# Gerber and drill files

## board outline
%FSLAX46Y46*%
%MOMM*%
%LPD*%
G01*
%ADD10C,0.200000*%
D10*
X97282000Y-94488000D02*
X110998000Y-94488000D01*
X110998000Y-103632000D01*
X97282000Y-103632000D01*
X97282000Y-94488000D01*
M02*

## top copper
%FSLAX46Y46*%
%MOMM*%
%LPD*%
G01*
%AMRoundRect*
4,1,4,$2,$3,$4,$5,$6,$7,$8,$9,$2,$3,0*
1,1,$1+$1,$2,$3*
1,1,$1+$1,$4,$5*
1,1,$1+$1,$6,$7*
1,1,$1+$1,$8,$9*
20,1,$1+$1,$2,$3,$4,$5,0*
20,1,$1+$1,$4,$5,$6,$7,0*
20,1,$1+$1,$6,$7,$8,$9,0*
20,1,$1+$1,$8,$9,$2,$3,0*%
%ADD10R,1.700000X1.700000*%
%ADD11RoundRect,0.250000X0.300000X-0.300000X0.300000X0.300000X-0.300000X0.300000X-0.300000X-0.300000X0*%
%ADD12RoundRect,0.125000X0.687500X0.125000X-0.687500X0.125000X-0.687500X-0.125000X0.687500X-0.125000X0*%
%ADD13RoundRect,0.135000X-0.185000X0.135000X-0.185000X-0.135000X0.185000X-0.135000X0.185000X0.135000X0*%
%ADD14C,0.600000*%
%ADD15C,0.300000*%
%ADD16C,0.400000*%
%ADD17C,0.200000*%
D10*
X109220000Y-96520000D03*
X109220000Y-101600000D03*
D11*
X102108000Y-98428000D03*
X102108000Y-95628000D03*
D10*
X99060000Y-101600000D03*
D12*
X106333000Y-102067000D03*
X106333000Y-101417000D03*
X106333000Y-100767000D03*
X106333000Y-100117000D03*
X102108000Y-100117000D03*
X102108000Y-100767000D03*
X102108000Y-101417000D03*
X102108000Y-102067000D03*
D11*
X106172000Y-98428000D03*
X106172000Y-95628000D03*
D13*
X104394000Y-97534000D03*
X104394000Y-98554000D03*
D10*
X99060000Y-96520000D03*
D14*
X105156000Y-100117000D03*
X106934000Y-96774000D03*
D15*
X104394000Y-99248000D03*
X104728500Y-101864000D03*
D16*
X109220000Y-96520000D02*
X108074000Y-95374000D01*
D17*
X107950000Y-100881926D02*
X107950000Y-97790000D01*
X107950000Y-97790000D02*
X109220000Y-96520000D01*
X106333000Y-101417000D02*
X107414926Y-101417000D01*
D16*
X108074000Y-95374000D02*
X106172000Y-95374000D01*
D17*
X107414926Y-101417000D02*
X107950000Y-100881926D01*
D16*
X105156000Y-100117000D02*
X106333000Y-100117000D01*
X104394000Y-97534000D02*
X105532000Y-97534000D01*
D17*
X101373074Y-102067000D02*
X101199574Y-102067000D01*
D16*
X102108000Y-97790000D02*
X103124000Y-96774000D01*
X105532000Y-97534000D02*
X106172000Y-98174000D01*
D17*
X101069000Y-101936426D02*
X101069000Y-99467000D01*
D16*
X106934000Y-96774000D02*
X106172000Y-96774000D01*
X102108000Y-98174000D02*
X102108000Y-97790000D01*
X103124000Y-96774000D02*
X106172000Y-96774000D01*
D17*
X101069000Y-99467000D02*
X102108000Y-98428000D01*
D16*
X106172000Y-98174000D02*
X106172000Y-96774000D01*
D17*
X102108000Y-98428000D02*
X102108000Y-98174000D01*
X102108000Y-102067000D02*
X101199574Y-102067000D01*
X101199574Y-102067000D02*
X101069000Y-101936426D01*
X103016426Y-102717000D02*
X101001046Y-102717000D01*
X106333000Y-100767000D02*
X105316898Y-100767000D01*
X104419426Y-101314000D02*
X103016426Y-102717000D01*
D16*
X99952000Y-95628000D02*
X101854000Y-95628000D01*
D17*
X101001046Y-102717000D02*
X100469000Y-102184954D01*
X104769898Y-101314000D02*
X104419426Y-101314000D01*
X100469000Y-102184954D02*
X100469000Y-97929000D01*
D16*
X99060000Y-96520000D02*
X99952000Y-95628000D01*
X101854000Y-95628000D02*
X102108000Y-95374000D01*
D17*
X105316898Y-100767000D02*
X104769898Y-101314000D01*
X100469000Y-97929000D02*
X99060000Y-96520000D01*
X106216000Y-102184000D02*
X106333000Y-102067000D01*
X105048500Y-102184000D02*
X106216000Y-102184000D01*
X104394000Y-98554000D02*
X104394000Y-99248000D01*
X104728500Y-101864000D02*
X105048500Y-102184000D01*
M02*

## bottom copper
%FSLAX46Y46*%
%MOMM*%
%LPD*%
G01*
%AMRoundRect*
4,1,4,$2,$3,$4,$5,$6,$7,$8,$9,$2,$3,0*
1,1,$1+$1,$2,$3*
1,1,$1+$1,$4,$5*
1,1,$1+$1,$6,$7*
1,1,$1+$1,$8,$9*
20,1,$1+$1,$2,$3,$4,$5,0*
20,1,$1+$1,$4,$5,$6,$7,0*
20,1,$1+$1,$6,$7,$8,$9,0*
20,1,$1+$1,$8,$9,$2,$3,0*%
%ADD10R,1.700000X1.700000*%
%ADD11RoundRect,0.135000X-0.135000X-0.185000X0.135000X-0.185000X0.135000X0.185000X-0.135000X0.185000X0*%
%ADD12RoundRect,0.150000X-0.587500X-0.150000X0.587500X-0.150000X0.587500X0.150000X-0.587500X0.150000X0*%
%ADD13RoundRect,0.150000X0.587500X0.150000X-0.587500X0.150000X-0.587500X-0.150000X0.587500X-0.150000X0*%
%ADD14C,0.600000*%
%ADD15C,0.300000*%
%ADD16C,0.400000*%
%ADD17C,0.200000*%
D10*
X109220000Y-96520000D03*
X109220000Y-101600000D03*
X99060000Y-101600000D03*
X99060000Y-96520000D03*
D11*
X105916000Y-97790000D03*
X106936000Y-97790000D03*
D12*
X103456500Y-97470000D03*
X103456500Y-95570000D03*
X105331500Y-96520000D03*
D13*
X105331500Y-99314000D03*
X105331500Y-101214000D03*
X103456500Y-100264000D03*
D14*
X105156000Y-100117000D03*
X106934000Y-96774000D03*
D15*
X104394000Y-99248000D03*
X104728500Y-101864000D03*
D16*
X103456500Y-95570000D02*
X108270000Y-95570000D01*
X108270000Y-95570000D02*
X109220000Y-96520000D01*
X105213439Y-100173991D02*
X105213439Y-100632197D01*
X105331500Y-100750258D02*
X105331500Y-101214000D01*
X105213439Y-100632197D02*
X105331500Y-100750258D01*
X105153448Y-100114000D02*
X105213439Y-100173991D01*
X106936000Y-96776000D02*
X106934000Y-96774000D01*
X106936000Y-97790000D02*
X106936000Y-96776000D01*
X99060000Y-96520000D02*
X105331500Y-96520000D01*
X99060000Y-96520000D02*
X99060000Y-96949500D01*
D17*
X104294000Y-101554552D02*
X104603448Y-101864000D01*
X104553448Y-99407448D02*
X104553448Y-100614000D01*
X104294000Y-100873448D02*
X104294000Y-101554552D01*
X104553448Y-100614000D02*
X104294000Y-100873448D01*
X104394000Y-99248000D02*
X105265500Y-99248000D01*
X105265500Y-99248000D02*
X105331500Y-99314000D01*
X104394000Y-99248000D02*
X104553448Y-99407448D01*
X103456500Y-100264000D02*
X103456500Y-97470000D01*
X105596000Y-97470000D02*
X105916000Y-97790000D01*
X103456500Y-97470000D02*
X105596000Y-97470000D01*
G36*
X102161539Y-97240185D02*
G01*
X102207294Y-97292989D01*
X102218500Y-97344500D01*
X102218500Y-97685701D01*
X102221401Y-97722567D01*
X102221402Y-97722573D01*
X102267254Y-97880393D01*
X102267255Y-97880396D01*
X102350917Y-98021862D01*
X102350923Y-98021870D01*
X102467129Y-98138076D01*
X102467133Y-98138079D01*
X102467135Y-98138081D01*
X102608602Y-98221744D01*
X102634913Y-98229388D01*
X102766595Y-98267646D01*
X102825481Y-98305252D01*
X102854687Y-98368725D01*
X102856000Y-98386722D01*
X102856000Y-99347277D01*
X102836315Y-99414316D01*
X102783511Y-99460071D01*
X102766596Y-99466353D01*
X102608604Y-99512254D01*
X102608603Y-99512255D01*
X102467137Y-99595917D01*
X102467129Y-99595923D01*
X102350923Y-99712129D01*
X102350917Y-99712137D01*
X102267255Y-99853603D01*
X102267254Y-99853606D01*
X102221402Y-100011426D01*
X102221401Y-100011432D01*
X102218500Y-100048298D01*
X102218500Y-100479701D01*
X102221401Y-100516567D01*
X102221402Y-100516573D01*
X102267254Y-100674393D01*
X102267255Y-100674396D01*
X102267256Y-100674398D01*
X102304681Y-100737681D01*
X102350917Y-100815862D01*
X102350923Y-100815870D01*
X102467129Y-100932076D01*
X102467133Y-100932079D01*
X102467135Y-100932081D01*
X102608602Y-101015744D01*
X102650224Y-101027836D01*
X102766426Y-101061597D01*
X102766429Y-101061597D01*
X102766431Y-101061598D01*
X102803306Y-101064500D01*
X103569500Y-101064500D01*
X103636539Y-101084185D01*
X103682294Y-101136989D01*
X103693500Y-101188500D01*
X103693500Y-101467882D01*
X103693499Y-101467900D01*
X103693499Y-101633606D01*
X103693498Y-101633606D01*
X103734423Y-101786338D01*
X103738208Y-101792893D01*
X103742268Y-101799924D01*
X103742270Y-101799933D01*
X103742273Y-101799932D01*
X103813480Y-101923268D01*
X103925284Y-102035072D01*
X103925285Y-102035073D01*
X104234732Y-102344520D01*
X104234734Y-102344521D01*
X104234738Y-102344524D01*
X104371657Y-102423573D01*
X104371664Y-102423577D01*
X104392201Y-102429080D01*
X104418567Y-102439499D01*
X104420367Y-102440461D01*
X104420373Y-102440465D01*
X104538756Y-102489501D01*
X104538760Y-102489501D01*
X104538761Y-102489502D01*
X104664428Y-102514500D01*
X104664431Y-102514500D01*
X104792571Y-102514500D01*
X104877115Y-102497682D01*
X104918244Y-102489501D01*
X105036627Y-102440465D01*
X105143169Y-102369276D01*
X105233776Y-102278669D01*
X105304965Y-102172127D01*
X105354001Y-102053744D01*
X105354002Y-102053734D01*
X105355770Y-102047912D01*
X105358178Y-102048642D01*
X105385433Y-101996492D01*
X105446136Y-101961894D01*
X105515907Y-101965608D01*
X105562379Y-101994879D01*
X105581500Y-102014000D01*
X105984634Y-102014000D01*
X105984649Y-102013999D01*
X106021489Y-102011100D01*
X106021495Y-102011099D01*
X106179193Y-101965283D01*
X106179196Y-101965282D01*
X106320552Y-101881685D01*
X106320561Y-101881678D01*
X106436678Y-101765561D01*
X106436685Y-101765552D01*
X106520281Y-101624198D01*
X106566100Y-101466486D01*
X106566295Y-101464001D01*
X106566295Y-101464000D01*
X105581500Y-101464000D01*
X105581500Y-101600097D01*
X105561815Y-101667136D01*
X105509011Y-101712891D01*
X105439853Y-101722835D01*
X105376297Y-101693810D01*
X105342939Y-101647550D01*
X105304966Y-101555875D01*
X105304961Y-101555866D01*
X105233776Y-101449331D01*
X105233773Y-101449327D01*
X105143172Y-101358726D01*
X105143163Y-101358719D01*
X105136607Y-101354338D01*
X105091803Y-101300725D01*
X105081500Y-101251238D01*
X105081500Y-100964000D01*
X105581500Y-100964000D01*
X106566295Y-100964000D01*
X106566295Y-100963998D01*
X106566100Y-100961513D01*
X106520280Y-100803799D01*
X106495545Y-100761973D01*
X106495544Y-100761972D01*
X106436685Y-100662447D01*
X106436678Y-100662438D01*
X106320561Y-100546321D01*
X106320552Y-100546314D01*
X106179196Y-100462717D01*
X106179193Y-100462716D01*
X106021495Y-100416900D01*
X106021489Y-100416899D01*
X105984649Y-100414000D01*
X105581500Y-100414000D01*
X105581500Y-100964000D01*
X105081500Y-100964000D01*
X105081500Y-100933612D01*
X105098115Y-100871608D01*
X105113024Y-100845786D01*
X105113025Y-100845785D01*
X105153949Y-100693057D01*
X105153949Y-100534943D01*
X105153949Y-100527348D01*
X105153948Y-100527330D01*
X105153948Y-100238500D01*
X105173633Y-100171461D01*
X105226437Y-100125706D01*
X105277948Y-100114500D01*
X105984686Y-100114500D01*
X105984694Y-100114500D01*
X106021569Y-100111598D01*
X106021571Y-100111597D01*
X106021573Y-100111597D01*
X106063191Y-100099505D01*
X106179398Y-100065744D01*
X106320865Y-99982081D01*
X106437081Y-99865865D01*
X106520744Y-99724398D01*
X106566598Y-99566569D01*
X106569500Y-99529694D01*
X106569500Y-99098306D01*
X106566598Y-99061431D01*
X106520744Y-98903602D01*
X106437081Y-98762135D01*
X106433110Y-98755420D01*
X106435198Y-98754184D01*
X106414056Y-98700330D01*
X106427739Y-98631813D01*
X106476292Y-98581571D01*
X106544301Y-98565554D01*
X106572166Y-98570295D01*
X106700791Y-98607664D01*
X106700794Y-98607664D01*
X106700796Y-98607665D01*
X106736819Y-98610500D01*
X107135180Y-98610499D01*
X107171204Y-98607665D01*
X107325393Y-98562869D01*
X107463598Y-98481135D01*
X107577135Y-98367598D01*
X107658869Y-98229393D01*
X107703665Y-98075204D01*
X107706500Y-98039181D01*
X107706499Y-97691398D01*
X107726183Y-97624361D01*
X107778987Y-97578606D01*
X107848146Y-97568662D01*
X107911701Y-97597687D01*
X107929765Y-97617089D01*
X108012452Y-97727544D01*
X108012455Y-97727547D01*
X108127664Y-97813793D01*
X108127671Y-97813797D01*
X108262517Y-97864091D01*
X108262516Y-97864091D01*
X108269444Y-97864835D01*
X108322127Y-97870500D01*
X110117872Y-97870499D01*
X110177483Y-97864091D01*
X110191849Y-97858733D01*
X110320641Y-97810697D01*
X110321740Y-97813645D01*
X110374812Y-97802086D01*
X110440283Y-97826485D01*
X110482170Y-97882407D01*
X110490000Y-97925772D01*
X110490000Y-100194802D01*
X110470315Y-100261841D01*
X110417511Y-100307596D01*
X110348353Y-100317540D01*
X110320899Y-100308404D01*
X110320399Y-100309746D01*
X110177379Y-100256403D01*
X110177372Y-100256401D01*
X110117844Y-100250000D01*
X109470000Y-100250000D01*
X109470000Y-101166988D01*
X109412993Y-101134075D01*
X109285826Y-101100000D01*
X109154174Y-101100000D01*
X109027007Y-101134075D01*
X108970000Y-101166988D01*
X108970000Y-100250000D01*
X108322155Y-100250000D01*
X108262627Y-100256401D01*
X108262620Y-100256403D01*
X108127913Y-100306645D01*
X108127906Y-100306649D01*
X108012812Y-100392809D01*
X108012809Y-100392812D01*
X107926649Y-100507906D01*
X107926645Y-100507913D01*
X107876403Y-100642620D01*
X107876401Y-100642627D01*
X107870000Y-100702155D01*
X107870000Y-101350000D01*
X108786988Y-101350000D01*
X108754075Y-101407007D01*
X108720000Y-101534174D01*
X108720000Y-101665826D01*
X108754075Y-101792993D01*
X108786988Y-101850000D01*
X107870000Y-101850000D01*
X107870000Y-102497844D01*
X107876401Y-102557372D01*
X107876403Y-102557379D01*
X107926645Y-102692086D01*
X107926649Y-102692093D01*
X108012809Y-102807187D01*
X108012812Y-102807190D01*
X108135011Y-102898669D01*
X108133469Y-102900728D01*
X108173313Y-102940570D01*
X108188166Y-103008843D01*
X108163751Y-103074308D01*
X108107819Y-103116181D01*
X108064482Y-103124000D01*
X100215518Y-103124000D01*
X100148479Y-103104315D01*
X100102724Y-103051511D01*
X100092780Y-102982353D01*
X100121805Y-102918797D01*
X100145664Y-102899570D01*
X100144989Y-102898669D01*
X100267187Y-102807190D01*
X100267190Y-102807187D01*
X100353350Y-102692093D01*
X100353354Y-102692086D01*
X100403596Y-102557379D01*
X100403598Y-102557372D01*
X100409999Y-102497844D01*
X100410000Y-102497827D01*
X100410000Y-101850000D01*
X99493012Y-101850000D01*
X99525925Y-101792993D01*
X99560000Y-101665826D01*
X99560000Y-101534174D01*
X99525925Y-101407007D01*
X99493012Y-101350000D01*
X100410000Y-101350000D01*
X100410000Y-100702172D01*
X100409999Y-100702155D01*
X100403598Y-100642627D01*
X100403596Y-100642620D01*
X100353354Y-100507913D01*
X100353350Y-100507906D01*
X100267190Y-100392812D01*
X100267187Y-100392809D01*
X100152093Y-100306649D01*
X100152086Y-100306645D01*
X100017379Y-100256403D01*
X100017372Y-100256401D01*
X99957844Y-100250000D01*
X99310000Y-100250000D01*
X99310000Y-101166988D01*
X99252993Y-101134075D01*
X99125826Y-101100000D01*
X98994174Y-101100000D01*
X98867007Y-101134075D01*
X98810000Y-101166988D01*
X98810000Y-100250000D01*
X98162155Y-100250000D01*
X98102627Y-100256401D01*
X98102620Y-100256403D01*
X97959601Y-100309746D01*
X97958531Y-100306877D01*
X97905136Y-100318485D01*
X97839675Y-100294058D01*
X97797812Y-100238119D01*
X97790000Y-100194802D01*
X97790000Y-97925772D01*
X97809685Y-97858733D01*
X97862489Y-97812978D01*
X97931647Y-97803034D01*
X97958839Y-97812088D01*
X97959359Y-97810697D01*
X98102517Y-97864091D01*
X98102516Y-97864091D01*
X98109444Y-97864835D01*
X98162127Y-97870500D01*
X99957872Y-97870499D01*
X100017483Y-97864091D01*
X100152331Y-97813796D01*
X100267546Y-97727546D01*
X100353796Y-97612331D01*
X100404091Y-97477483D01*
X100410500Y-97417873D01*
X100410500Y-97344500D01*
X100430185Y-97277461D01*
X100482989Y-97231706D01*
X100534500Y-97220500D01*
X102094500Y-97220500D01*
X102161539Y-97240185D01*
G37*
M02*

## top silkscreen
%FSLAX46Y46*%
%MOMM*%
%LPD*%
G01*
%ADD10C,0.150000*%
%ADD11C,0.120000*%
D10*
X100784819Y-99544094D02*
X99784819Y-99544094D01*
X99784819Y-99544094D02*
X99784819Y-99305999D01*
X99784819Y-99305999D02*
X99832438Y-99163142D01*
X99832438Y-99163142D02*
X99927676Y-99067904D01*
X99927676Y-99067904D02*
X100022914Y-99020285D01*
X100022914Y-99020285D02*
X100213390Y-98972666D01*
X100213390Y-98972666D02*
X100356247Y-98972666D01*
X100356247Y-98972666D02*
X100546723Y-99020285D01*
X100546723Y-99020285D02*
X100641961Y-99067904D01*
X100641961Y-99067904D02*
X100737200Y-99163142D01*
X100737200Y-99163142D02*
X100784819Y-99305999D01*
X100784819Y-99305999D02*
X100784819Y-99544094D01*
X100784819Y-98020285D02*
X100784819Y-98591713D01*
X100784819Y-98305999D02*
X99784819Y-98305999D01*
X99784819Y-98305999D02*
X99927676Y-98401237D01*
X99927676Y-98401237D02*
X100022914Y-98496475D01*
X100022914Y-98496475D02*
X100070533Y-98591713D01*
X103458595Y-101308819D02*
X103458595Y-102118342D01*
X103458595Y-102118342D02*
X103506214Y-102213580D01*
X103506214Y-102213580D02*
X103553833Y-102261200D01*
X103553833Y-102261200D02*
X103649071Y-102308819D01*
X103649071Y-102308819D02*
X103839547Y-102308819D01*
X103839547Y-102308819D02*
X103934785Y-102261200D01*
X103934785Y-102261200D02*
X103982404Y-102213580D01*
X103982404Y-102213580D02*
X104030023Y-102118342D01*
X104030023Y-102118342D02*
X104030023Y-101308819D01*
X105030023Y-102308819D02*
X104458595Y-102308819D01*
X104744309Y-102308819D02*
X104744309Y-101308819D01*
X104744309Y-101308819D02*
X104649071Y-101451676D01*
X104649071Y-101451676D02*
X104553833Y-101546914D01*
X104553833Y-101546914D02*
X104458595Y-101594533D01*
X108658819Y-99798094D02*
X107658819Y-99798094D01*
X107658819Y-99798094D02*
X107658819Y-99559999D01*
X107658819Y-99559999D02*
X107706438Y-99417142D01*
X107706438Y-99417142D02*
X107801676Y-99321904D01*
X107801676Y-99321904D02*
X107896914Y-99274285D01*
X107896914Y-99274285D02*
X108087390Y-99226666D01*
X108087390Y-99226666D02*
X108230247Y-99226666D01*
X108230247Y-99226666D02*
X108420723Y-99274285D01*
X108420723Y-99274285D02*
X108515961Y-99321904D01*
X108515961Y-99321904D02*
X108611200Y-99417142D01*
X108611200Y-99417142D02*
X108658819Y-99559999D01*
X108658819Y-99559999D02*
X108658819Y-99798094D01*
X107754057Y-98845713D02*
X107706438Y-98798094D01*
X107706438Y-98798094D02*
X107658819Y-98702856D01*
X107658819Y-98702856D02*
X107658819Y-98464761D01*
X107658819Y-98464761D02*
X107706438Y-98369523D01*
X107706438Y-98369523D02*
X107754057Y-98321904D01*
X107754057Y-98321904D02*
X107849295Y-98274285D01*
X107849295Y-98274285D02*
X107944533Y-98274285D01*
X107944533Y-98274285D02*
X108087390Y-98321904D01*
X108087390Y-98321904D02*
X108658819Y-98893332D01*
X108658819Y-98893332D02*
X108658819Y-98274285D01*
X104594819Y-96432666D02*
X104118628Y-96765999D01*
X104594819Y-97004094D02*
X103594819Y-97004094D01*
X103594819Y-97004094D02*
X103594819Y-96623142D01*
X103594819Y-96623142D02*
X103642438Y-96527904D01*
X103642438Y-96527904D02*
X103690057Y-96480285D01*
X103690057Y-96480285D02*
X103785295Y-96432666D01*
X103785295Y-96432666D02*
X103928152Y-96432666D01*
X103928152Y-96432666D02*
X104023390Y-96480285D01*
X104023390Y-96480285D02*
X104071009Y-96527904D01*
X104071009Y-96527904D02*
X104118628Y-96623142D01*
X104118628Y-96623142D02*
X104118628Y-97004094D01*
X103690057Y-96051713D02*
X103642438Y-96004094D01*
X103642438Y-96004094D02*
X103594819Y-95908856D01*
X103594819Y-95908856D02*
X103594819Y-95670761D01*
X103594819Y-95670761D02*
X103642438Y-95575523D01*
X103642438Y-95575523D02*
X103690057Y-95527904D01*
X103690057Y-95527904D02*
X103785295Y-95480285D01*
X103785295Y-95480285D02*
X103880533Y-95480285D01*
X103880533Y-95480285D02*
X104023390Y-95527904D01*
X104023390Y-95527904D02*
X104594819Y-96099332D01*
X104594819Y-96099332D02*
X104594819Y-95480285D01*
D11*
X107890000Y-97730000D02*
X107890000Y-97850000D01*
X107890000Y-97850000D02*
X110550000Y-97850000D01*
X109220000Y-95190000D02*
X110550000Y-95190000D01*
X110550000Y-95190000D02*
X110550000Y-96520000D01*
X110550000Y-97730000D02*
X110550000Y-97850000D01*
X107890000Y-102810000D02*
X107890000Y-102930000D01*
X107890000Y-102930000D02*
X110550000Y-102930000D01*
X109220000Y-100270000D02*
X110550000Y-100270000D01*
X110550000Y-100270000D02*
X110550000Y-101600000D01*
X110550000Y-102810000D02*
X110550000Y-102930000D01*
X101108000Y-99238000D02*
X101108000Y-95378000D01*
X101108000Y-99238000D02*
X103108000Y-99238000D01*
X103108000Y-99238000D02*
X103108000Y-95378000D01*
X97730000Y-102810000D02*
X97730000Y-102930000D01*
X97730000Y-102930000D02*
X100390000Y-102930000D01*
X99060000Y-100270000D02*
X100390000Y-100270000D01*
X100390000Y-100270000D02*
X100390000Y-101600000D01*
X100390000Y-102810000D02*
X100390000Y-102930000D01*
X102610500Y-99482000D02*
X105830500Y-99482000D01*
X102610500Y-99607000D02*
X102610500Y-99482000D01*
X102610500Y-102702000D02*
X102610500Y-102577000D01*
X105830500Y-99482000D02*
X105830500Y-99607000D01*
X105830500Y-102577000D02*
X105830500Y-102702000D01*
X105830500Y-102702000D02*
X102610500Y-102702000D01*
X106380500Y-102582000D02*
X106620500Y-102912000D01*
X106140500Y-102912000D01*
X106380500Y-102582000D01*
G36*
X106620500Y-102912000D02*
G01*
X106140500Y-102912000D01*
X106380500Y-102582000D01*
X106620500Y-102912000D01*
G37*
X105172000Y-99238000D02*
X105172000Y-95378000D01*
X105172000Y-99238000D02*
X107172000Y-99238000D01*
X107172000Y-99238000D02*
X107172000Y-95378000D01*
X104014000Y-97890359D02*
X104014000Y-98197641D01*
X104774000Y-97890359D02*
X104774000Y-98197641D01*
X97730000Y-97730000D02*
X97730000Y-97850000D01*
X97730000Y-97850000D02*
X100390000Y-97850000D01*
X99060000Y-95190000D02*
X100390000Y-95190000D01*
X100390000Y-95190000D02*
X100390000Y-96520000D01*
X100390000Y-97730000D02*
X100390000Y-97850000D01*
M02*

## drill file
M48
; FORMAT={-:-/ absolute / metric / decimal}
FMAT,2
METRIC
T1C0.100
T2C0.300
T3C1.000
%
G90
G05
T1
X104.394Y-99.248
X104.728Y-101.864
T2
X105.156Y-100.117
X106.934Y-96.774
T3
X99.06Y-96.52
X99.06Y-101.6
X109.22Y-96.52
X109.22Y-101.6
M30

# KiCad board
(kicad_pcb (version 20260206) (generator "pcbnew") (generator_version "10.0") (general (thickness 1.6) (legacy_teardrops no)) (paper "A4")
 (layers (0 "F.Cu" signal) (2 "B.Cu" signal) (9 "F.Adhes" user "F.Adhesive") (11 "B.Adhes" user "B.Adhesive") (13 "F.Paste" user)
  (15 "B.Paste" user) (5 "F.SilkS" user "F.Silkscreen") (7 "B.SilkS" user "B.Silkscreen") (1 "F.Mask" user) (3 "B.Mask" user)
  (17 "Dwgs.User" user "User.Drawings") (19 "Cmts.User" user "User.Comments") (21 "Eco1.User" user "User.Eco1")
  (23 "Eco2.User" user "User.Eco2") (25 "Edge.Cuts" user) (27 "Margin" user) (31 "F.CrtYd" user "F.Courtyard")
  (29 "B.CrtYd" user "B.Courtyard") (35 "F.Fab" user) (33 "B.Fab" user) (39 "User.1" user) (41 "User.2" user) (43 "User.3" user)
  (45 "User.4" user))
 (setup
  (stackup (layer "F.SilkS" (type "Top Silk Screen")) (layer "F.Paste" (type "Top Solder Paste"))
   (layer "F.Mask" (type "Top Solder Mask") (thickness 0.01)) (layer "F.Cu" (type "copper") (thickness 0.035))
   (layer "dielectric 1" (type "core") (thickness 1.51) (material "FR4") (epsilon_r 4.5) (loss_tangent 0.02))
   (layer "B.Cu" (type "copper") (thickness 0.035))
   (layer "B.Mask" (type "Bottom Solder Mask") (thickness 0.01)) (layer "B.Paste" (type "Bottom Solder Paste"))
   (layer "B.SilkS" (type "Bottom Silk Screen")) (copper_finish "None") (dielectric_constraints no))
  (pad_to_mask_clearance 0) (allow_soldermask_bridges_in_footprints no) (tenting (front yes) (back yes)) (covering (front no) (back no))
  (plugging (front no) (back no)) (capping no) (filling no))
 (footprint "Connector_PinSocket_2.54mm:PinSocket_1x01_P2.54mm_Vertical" (layer "F.Cu") (at 109.22 96.52)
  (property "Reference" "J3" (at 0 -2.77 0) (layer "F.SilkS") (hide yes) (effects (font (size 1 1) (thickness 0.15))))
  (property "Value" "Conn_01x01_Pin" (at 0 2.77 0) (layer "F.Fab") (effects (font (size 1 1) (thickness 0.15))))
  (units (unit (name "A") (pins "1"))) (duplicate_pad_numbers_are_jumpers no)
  (fp_line (start -1.33 1.21) (end -1.33 1.33) (stroke (width 0.12) (type solid)) (layer "F.SilkS"))
  (fp_line (start -1.33 1.33) (end 1.33 1.33) (stroke (width 0.12) (type solid)) (layer "F.SilkS"))
  (fp_line (start 0 -1.33) (end 1.33 -1.33) (stroke (width 0.12) (type solid)) (layer "F.SilkS"))
  (fp_line (start 1.33 -1.33) (end 1.33 0) (stroke (width 0.12) (type solid)) (layer "F.SilkS"))
  (fp_line (start 1.33 1.21) (end 1.33 1.33) (stroke (width 0.12) (type solid)) (layer "F.SilkS"))
  (pad "1" thru_hole rect (at 0 0) (size 1.7 1.7) (drill 1) (layers "*.Cu" "*.Mask") (remove_unused_layers no) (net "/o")))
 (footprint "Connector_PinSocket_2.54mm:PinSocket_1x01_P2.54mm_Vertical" (layer "F.Cu") (at 109.22 101.6)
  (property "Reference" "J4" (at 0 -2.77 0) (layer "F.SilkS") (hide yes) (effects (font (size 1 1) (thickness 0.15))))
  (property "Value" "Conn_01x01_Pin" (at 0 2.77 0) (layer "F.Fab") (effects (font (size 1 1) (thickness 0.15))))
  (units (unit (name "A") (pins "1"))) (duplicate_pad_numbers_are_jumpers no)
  (fp_line (start -1.33 1.21) (end -1.33 1.33) (stroke (width 0.12) (type solid)) (layer "F.SilkS"))
  (fp_line (start -1.33 1.33) (end 1.33 1.33) (stroke (width 0.12) (type solid)) (layer "F.SilkS"))
  (fp_line (start 0 -1.33) (end 1.33 -1.33) (stroke (width 0.12) (type solid)) (layer "F.SilkS"))
  (fp_line (start 1.33 -1.33) (end 1.33 0) (stroke (width 0.12) (type solid)) (layer "F.SilkS"))
  (fp_line (start 1.33 1.21) (end 1.33 1.33) (stroke (width 0.12) (type solid)) (layer "F.SilkS"))
  (pad "1" thru_hole rect (at 0 0) (size 1.7 1.7) (drill 1) (layers "*.Cu" "*.Mask") (remove_unused_layers no) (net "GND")))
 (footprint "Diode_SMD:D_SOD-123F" (layer "F.Cu") (at 102.108 97.028 90)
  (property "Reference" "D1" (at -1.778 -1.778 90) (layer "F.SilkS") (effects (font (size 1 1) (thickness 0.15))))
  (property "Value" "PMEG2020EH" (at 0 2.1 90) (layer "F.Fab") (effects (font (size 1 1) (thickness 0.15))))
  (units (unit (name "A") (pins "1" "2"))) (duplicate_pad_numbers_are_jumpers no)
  (fp_line (start -2.21 -1) (end 1.65 -1) (stroke (width 0.12) (type solid)) (layer "F.SilkS"))
  (fp_line (start -2.21 -1) (end -2.21 1) (stroke (width 0.12) (type solid)) (layer "F.SilkS"))
  (fp_line (start -2.21 1) (end 1.65 1) (stroke (width 0.12) (type solid)) (layer "F.SilkS"))
  (pad "1" smd roundrect (at -1.4 0 90) (size 1.1 1.1) (layers "F.Cu" "F.Mask" "F.Paste") (roundrect_rratio 0.2272727273) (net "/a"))
  (pad "2" smd roundrect (at 1.4 0 90) (size 1.1 1.1) (layers "F.Cu" "F.Mask" "F.Paste") (roundrect_rratio 0.2272727273) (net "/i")))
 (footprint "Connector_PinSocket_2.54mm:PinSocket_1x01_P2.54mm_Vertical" (layer "F.Cu") (at 99.06 101.6)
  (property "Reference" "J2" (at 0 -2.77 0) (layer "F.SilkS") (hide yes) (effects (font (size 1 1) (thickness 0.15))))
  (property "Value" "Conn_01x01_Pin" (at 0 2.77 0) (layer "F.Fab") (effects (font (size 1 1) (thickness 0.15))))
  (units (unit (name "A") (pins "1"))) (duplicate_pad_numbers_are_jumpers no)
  (fp_line (start -1.33 1.21) (end -1.33 1.33) (stroke (width 0.12) (type solid)) (layer "F.SilkS"))
  (fp_line (start -1.33 1.33) (end 1.33 1.33) (stroke (width 0.12) (type solid)) (layer "F.SilkS"))
  (fp_line (start 0 -1.33) (end 1.33 -1.33) (stroke (width 0.12) (type solid)) (layer "F.SilkS"))
  (fp_line (start 1.33 -1.33) (end 1.33 0) (stroke (width 0.12) (type solid)) (layer "F.SilkS"))
  (fp_line (start 1.33 1.21) (end 1.33 1.33) (stroke (width 0.12) (type solid)) (layer "F.SilkS"))
  (pad "1" thru_hole rect (at 0 0) (size 1.7 1.7) (drill 1) (layers "*.Cu" "*.Mask") (remove_unused_layers no) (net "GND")))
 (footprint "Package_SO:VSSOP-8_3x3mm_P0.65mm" (layer "F.Cu") (at 104.2205 101.092 180)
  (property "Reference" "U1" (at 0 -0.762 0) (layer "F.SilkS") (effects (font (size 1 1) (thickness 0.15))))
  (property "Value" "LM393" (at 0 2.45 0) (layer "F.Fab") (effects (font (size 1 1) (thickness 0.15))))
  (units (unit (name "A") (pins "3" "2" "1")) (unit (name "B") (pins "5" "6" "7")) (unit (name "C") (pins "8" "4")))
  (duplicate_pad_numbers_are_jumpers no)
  (fp_line (start 1.61 1.61) (end -1.61 1.61) (stroke (width 0.12) (type solid)) (layer "F.SilkS"))
  (fp_line (start 1.61 1.485) (end 1.61 1.61) (stroke (width 0.12) (type solid)) (layer "F.SilkS"))
  (fp_line (start 1.61 -1.61) (end 1.61 -1.485) (stroke (width 0.12) (type solid)) (layer "F.SilkS"))
  (fp_line (start -1.61 1.61) (end -1.61 1.485) (stroke (width 0.12) (type solid)) (layer "F.SilkS"))
  (fp_line (start -1.61 -1.485) (end -1.61 -1.61) (stroke (width 0.12) (type solid)) (layer "F.SilkS"))
  (fp_line (start -1.61 -1.61) (end 1.61 -1.61) (stroke (width 0.12) (type solid)) (layer "F.SilkS"))
  (fp_poly (pts (xy -2.16 -1.49) (xy -2.4 -1.82) (xy -1.92 -1.82)) (stroke (width 0.12) (type solid)) (fill yes) (layer "F.SilkS"))
  (pad "1" smd roundrect (at -2.1125 -0.975 180) (size 1.625 0.5) (layers "F.Cu" "F.Mask" "F.Paste") (roundrect_rratio 0.25)
   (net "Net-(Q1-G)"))
  (pad "2" smd roundrect (at -2.1125 -0.325 180) (size 1.625 0.5) (layers "F.Cu" "F.Mask" "F.Paste") (roundrect_rratio 0.25) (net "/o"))
  (pad "3" smd roundrect (at -2.1125 0.325 180) (size 1.625 0.5) (layers "F.Cu" "F.Mask" "F.Paste") (roundrect_rratio 0.25) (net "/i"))
  (pad "4" smd roundrect (at -2.1125 0.975 180) (size 1.625 0.5) (layers "F.Cu" "F.Mask" "F.Paste") (roundrect_rratio 0.25) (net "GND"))
  (pad "5" smd roundrect (at 2.1125 0.975 180) (size 1.625 0.5) (layers "F.Cu" "F.Mask" "F.Paste") (roundrect_rratio 0.25)
   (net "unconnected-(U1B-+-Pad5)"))
  (pad "6" smd roundrect (at 2.1125 0.325 180) (size 1.625 0.5) (layers "F.Cu" "F.Mask" "F.Paste") (roundrect_rratio 0.25)
   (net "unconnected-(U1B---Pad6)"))
  (pad "7" smd roundrect (at 2.1125 -0.325 180) (size 1.625 0.5) (layers "F.Cu" "F.Mask" "F.Paste") (roundrect_rratio 0.25)
   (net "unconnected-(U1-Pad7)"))
  (pad "8" smd roundrect (at 2.1125 -0.975 180) (size 1.625 0.5) (layers "F.Cu" "F.Mask" "F.Paste") (roundrect_rratio 0.25) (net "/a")))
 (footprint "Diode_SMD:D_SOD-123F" (layer "F.Cu") (at 106.172 97.028 90)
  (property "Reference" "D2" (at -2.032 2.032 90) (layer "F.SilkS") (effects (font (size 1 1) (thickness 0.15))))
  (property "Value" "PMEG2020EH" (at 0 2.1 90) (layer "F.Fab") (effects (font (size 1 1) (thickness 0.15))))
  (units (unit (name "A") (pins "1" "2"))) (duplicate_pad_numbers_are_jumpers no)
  (fp_line (start -2.21 -1) (end 1.65 -1) (stroke (width 0.12) (type solid)) (layer "F.SilkS"))
  (fp_line (start -2.21 -1) (end -2.21 1) (stroke (width 0.12) (type solid)) (layer "F.SilkS"))
  (fp_line (start -2.21 1) (end 1.65 1) (stroke (width 0.12) (type solid)) (layer "F.SilkS"))
  (pad "1" smd roundrect (at -1.4 0 90) (size 1.1 1.1) (layers "F.Cu" "F.Mask" "F.Paste") (roundrect_rratio 0.2272727273) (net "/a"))
  (pad "2" smd roundrect (at 1.4 0 90) (size 1.1 1.1) (layers "F.Cu" "F.Mask" "F.Paste") (roundrect_rratio 0.2272727273) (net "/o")))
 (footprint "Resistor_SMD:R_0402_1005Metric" (layer "F.Cu") (at 104.394 98.044 -90)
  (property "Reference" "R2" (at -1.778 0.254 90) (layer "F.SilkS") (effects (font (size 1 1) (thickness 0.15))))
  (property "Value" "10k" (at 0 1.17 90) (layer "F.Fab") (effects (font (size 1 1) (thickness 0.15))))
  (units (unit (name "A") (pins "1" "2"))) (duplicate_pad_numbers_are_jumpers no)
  (fp_line (start -0.153641 0.38) (end 0.153641 0.38) (stroke (width 0.12) (type solid)) (layer "F.SilkS"))
  (fp_line (start -0.153641 -0.38) (end 0.153641 -0.38) (stroke (width 0.12) (type solid)) (layer "F.SilkS"))
  (pad "1" smd roundrect (at -0.51 0 270) (size 0.54 0.64) (layers "F.Cu" "F.Mask" "F.Paste") (roundrect_rratio 0.25) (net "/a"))
  (pad "2" smd roundrect (at 0.51 0 270) (size 0.54 0.64) (layers "F.Cu" "F.Mask" "F.Paste") (roundrect_rratio 0.25) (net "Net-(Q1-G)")))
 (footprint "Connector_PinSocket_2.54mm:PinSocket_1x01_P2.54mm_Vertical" (layer "F.Cu") (at 99.06 96.52)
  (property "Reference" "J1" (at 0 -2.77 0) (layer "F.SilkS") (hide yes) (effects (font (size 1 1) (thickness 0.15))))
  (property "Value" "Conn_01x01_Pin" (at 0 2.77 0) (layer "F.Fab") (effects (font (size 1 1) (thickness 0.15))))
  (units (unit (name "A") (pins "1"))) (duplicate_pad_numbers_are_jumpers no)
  (fp_line (start -1.33 1.21) (end -1.33 1.33) (stroke (width 0.12) (type solid)) (layer "F.SilkS"))
  (fp_line (start -1.33 1.33) (end 1.33 1.33) (stroke (width 0.12) (type solid)) (layer "F.SilkS"))
  (fp_line (start 0 -1.33) (end 1.33 -1.33) (stroke (width 0.12) (type solid)) (layer "F.SilkS"))
  (fp_line (start 1.33 -1.33) (end 1.33 0) (stroke (width 0.12) (type solid)) (layer "F.SilkS"))
  (fp_line (start 1.33 1.21) (end 1.33 1.33) (stroke (width 0.12) (type solid)) (layer "F.SilkS"))
  (pad "1" thru_hole rect (at 0 0) (size 1.7 1.7) (drill 1) (layers "*.Cu" "*.Mask") (remove_unused_layers no) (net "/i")))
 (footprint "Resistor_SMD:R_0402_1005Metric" (layer "B.Cu") (at 106.426 97.79)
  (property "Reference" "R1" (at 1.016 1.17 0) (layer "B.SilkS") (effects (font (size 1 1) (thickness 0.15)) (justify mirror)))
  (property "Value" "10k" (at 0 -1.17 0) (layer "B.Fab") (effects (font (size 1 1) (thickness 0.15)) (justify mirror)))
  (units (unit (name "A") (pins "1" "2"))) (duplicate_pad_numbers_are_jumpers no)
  (pad "1" smd roundrect (at -0.51 0) (size 0.54 0.64) (layers "B.Cu" "B.Mask" "B.Paste") (roundrect_rratio 0.25) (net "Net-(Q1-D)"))
  (pad "2" smd roundrect (at 0.51 0) (size 0.54 0.64) (layers "B.Cu" "B.Mask" "B.Paste") (roundrect_rratio 0.25) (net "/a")))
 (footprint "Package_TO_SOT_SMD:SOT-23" (layer "B.Cu") (at 104.394 96.52)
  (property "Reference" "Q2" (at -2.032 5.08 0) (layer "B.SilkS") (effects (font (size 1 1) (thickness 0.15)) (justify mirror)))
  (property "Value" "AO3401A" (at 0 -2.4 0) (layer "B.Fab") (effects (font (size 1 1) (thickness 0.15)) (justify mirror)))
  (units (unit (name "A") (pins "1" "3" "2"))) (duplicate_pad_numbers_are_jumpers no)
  (pad "1" smd roundrect (at -0.9375 0.95) (size 1.475 0.6) (layers "B.Cu" "B.Mask" "B.Paste") (roundrect_rratio 0.25) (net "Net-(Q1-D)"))
  (pad "2" smd roundrect (at -0.9375 -0.95) (size 1.475 0.6) (layers "B.Cu" "B.Mask" "B.Paste") (roundrect_rratio 0.25) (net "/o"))
  (pad "3" smd roundrect (at 0.9375 0) (size 1.475 0.6) (layers "B.Cu" "B.Mask" "B.Paste") (roundrect_rratio 0.25) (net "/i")))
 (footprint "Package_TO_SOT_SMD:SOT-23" (layer "B.Cu") (at 104.394 100.264 180)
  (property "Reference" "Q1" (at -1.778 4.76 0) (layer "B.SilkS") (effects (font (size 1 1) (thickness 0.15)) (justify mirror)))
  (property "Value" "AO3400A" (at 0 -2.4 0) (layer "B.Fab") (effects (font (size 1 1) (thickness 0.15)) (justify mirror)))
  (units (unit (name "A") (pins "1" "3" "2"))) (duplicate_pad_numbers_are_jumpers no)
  (pad "1" smd roundrect (at -0.9375 0.95 180) (size 1.475 0.6) (layers "B.Cu" "B.Mask" "B.Paste") (roundrect_rratio 0.25)
   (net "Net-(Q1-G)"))
  (pad "2" smd roundrect (at -0.9375 -0.95 180) (size 1.475 0.6) (layers "B.Cu" "B.Mask" "B.Paste") (roundrect_rratio 0.25) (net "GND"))
  (pad "3" smd roundrect (at 0.9375 0 180) (size 1.475 0.6) (layers "B.Cu" "B.Mask" "B.Paste") (roundrect_rratio 0.25) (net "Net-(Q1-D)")))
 (gr_rect (start 97.282 94.488) (end 110.998 103.632) (stroke (width 0.2) (type solid)) (fill no) (layer "Edge.Cuts"))
 (segment (start 109.22 96.52) (end 108.074 95.374) (width 0.4) (layer "F.Cu") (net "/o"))
 (segment (start 107.95 100.881926) (end 107.95 97.79) (width 0.2) (layer "F.Cu") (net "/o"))
 (segment (start 107.95 97.79) (end 109.22 96.52) (width 0.2) (layer "F.Cu") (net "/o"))
 (segment (start 106.333 101.417) (end 107.414926 101.417) (width 0.2) (layer "F.Cu") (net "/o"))
 (segment (start 108.074 95.374) (end 106.172 95.374) (width 0.4) (layer "F.Cu") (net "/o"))
 (segment (start 107.414926 101.417) (end 107.95 100.881926) (width 0.2) (layer "F.Cu") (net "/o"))
 (segment (start 103.4565 95.57) (end 108.27 95.57) (width 0.4) (layer "B.Cu") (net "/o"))
 (segment (start 108.27 95.57) (end 109.22 96.52) (width 0.4) (layer "B.Cu") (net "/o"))
 (segment (start 105.156 100.117) (end 106.333 100.117) (width 0.4) (layer "F.Cu") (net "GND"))
 (via (at 105.156 100.117) (size 0.6) (drill 0.3) (layers "F.Cu" "B.Cu") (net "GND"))
 (segment (start 105.213439 100.173991) (end 105.213439 100.632197) (width 0.4) (layer "B.Cu") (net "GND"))
 (segment (start 105.3315 100.750258) (end 105.3315 101.214) (width 0.4) (layer "B.Cu") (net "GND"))
 (segment (start 105.213439 100.632197) (end 105.3315 100.750258) (width 0.4) (layer "B.Cu") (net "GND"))
 (segment (start 105.153448 100.114) (end 105.213439 100.173991) (width 0.4) (layer "B.Cu") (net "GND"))
 (segment (start 104.394 97.534) (end 105.532 97.534) (width 0.4) (layer "F.Cu") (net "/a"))
 (segment (start 101.373074 102.067) (end 101.199574 102.067) (width 0.2) (layer "F.Cu") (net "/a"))
 (segment (start 102.108 97.79) (end 103.124 96.774) (width 0.4) (layer "F.Cu") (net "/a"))
 (segment (start 105.532 97.534) (end 106.172 98.174) (width 0.4) (layer "F.Cu") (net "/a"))
 (segment (start 101.069 101.936426) (end 101.069 99.467) (width 0.2) (layer "F.Cu") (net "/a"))
 (segment (start 106.934 96.774) (end 106.172 96.774) (width 0.4) (layer "F.Cu") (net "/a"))
 (segment (start 102.108 98.174) (end 102.108 97.79) (width 0.4) (layer "F.Cu") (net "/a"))
 (segment (start 103.124 96.774) (end 106.172 96.774) (width 0.4) (layer "F.Cu") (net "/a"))
 (segment (start 101.069 99.467) (end 102.108 98.428) (width 0.2) (layer "F.Cu") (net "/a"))
 (segment (start 106.172 98.174) (end 106.172 96.774) (width 0.4) (layer "F.Cu") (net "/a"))
 (segment (start 102.108 98.428) (end 102.108 98.174) (width 0.2) (layer "F.Cu") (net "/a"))
 (segment (start 102.108 102.067) (end 101.199574 102.067) (width 0.2) (layer "F.Cu") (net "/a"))
 (segment (start 101.199574 102.067) (end 101.069 101.936426) (width 0.2) (layer "F.Cu") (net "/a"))
 (via (at 106.934 96.774) (size 0.6) (drill 0.3) (layers "F.Cu" "B.Cu") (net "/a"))
 (segment (start 106.936 96.776) (end 106.934 96.774) (width 0.4) (layer "B.Cu") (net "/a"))
 (segment (start 106.936 97.79) (end 106.936 96.776) (width 0.4) (layer "B.Cu") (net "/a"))
 (segment (start 103.016426 102.717) (end 101.001046 102.717) (width 0.2) (layer "F.Cu") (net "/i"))
 (segment (start 106.333 100.767) (end 105.316898 100.767) (width 0.2) (layer "F.Cu") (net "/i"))
 (segment (start 104.419426 101.314) (end 103.016426 102.717) (width 0.2) (layer "F.Cu") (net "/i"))
 (segment (start 99.952 95.628) (end 101.854 95.628) (width 0.4) (layer "F.Cu") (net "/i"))
 (segment (start 101.001046 102.717) (end 100.469 102.184954) (width 0.2) (layer "F.Cu") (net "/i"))
 (segment (start 104.769898 101.314) (end 104.419426 101.314) (width 0.2) (layer "F.Cu") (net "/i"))
 (segment (start 100.469 102.184954) (end 100.469 97.929) (width 0.2) (layer "F.Cu") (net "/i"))
 (segment (start 99.06 96.52) (end 99.952 95.628) (width 0.4) (layer "F.Cu") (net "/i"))
 (segment (start 101.854 95.628) (end 102.108 95.374) (width 0.4) (layer "F.Cu") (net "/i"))
 (segment (start 105.316898 100.767) (end 104.769898 101.314) (width 0.2) (layer "F.Cu") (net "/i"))
 (segment (start 100.469 97.929) (end 99.06 96.52) (width 0.2) (layer "F.Cu") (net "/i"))
 (segment (start 99.06 96.52) (end 105.3315 96.52) (width 0.4) (layer "B.Cu") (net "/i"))
 (segment (start 99.06 96.52) (end 99.06 96.9495) (width 0.4) (layer "B.Cu") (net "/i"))
 (segment (start 106.216 102.184) (end 106.333 102.067) (width 0.2) (layer "F.Cu") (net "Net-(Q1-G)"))
 (segment (start 105.0485 102.184) (end 106.216 102.184) (width 0.2) (layer "F.Cu") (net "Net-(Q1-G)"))
 (segment (start 104.394 98.554) (end 104.394 99.248) (width 0.2) (layer "F.Cu") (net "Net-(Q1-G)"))
 (segment (start 104.7285 101.864) (end 105.0485 102.184) (width 0.2) (layer "F.Cu") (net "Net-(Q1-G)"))
 (via micro (at 104.394 99.248) (size 0.3) (drill 0.1) (layers "F.Cu" "B.Cu") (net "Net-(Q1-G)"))
 (via micro (at 104.7285 101.864) (size 0.3) (drill 0.1) (layers "F.Cu" "B.Cu") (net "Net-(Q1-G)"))
 (segment (start 104.294 101.554552) (end 104.603448 101.864) (width 0.2) (layer "B.Cu") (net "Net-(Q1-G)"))
 (segment (start 104.553448 99.407448) (end 104.553448 100.614) (width 0.2) (layer "B.Cu") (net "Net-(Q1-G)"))
 (segment (start 104.294 100.873448) (end 104.294 101.554552) (width 0.2) (layer "B.Cu") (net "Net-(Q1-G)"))
 (segment (start 104.553448 100.614) (end 104.294 100.873448) (width 0.2) (layer "B.Cu") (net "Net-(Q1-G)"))
 (segment (start 104.394 99.248) (end 105.2655 99.248) (width 0.2) (layer "B.Cu") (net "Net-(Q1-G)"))
 (segment (start 105.2655 99.248) (end 105.3315 99.314) (width 0.2) (layer "B.Cu") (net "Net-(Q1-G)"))
 (segment (start 104.394 99.248) (end 104.553448 99.407448) (width 0.2) (layer "B.Cu") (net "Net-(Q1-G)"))
 (segment (start 103.4565 100.264) (end 103.4565 97.47) (width 0.2) (layer "B.Cu") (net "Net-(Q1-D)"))
 (segment (start 105.596 97.47) (end 105.916 97.79) (width 0.2) (layer "B.Cu") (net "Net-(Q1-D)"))
 (segment (start 103.4565 97.47) (end 105.596 97.47) (width 0.2) (layer "B.Cu") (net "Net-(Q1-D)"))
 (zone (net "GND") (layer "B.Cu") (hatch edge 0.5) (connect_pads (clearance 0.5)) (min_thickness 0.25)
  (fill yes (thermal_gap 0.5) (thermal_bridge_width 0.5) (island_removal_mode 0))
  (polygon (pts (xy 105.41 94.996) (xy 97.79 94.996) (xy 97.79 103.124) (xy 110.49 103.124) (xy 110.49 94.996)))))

